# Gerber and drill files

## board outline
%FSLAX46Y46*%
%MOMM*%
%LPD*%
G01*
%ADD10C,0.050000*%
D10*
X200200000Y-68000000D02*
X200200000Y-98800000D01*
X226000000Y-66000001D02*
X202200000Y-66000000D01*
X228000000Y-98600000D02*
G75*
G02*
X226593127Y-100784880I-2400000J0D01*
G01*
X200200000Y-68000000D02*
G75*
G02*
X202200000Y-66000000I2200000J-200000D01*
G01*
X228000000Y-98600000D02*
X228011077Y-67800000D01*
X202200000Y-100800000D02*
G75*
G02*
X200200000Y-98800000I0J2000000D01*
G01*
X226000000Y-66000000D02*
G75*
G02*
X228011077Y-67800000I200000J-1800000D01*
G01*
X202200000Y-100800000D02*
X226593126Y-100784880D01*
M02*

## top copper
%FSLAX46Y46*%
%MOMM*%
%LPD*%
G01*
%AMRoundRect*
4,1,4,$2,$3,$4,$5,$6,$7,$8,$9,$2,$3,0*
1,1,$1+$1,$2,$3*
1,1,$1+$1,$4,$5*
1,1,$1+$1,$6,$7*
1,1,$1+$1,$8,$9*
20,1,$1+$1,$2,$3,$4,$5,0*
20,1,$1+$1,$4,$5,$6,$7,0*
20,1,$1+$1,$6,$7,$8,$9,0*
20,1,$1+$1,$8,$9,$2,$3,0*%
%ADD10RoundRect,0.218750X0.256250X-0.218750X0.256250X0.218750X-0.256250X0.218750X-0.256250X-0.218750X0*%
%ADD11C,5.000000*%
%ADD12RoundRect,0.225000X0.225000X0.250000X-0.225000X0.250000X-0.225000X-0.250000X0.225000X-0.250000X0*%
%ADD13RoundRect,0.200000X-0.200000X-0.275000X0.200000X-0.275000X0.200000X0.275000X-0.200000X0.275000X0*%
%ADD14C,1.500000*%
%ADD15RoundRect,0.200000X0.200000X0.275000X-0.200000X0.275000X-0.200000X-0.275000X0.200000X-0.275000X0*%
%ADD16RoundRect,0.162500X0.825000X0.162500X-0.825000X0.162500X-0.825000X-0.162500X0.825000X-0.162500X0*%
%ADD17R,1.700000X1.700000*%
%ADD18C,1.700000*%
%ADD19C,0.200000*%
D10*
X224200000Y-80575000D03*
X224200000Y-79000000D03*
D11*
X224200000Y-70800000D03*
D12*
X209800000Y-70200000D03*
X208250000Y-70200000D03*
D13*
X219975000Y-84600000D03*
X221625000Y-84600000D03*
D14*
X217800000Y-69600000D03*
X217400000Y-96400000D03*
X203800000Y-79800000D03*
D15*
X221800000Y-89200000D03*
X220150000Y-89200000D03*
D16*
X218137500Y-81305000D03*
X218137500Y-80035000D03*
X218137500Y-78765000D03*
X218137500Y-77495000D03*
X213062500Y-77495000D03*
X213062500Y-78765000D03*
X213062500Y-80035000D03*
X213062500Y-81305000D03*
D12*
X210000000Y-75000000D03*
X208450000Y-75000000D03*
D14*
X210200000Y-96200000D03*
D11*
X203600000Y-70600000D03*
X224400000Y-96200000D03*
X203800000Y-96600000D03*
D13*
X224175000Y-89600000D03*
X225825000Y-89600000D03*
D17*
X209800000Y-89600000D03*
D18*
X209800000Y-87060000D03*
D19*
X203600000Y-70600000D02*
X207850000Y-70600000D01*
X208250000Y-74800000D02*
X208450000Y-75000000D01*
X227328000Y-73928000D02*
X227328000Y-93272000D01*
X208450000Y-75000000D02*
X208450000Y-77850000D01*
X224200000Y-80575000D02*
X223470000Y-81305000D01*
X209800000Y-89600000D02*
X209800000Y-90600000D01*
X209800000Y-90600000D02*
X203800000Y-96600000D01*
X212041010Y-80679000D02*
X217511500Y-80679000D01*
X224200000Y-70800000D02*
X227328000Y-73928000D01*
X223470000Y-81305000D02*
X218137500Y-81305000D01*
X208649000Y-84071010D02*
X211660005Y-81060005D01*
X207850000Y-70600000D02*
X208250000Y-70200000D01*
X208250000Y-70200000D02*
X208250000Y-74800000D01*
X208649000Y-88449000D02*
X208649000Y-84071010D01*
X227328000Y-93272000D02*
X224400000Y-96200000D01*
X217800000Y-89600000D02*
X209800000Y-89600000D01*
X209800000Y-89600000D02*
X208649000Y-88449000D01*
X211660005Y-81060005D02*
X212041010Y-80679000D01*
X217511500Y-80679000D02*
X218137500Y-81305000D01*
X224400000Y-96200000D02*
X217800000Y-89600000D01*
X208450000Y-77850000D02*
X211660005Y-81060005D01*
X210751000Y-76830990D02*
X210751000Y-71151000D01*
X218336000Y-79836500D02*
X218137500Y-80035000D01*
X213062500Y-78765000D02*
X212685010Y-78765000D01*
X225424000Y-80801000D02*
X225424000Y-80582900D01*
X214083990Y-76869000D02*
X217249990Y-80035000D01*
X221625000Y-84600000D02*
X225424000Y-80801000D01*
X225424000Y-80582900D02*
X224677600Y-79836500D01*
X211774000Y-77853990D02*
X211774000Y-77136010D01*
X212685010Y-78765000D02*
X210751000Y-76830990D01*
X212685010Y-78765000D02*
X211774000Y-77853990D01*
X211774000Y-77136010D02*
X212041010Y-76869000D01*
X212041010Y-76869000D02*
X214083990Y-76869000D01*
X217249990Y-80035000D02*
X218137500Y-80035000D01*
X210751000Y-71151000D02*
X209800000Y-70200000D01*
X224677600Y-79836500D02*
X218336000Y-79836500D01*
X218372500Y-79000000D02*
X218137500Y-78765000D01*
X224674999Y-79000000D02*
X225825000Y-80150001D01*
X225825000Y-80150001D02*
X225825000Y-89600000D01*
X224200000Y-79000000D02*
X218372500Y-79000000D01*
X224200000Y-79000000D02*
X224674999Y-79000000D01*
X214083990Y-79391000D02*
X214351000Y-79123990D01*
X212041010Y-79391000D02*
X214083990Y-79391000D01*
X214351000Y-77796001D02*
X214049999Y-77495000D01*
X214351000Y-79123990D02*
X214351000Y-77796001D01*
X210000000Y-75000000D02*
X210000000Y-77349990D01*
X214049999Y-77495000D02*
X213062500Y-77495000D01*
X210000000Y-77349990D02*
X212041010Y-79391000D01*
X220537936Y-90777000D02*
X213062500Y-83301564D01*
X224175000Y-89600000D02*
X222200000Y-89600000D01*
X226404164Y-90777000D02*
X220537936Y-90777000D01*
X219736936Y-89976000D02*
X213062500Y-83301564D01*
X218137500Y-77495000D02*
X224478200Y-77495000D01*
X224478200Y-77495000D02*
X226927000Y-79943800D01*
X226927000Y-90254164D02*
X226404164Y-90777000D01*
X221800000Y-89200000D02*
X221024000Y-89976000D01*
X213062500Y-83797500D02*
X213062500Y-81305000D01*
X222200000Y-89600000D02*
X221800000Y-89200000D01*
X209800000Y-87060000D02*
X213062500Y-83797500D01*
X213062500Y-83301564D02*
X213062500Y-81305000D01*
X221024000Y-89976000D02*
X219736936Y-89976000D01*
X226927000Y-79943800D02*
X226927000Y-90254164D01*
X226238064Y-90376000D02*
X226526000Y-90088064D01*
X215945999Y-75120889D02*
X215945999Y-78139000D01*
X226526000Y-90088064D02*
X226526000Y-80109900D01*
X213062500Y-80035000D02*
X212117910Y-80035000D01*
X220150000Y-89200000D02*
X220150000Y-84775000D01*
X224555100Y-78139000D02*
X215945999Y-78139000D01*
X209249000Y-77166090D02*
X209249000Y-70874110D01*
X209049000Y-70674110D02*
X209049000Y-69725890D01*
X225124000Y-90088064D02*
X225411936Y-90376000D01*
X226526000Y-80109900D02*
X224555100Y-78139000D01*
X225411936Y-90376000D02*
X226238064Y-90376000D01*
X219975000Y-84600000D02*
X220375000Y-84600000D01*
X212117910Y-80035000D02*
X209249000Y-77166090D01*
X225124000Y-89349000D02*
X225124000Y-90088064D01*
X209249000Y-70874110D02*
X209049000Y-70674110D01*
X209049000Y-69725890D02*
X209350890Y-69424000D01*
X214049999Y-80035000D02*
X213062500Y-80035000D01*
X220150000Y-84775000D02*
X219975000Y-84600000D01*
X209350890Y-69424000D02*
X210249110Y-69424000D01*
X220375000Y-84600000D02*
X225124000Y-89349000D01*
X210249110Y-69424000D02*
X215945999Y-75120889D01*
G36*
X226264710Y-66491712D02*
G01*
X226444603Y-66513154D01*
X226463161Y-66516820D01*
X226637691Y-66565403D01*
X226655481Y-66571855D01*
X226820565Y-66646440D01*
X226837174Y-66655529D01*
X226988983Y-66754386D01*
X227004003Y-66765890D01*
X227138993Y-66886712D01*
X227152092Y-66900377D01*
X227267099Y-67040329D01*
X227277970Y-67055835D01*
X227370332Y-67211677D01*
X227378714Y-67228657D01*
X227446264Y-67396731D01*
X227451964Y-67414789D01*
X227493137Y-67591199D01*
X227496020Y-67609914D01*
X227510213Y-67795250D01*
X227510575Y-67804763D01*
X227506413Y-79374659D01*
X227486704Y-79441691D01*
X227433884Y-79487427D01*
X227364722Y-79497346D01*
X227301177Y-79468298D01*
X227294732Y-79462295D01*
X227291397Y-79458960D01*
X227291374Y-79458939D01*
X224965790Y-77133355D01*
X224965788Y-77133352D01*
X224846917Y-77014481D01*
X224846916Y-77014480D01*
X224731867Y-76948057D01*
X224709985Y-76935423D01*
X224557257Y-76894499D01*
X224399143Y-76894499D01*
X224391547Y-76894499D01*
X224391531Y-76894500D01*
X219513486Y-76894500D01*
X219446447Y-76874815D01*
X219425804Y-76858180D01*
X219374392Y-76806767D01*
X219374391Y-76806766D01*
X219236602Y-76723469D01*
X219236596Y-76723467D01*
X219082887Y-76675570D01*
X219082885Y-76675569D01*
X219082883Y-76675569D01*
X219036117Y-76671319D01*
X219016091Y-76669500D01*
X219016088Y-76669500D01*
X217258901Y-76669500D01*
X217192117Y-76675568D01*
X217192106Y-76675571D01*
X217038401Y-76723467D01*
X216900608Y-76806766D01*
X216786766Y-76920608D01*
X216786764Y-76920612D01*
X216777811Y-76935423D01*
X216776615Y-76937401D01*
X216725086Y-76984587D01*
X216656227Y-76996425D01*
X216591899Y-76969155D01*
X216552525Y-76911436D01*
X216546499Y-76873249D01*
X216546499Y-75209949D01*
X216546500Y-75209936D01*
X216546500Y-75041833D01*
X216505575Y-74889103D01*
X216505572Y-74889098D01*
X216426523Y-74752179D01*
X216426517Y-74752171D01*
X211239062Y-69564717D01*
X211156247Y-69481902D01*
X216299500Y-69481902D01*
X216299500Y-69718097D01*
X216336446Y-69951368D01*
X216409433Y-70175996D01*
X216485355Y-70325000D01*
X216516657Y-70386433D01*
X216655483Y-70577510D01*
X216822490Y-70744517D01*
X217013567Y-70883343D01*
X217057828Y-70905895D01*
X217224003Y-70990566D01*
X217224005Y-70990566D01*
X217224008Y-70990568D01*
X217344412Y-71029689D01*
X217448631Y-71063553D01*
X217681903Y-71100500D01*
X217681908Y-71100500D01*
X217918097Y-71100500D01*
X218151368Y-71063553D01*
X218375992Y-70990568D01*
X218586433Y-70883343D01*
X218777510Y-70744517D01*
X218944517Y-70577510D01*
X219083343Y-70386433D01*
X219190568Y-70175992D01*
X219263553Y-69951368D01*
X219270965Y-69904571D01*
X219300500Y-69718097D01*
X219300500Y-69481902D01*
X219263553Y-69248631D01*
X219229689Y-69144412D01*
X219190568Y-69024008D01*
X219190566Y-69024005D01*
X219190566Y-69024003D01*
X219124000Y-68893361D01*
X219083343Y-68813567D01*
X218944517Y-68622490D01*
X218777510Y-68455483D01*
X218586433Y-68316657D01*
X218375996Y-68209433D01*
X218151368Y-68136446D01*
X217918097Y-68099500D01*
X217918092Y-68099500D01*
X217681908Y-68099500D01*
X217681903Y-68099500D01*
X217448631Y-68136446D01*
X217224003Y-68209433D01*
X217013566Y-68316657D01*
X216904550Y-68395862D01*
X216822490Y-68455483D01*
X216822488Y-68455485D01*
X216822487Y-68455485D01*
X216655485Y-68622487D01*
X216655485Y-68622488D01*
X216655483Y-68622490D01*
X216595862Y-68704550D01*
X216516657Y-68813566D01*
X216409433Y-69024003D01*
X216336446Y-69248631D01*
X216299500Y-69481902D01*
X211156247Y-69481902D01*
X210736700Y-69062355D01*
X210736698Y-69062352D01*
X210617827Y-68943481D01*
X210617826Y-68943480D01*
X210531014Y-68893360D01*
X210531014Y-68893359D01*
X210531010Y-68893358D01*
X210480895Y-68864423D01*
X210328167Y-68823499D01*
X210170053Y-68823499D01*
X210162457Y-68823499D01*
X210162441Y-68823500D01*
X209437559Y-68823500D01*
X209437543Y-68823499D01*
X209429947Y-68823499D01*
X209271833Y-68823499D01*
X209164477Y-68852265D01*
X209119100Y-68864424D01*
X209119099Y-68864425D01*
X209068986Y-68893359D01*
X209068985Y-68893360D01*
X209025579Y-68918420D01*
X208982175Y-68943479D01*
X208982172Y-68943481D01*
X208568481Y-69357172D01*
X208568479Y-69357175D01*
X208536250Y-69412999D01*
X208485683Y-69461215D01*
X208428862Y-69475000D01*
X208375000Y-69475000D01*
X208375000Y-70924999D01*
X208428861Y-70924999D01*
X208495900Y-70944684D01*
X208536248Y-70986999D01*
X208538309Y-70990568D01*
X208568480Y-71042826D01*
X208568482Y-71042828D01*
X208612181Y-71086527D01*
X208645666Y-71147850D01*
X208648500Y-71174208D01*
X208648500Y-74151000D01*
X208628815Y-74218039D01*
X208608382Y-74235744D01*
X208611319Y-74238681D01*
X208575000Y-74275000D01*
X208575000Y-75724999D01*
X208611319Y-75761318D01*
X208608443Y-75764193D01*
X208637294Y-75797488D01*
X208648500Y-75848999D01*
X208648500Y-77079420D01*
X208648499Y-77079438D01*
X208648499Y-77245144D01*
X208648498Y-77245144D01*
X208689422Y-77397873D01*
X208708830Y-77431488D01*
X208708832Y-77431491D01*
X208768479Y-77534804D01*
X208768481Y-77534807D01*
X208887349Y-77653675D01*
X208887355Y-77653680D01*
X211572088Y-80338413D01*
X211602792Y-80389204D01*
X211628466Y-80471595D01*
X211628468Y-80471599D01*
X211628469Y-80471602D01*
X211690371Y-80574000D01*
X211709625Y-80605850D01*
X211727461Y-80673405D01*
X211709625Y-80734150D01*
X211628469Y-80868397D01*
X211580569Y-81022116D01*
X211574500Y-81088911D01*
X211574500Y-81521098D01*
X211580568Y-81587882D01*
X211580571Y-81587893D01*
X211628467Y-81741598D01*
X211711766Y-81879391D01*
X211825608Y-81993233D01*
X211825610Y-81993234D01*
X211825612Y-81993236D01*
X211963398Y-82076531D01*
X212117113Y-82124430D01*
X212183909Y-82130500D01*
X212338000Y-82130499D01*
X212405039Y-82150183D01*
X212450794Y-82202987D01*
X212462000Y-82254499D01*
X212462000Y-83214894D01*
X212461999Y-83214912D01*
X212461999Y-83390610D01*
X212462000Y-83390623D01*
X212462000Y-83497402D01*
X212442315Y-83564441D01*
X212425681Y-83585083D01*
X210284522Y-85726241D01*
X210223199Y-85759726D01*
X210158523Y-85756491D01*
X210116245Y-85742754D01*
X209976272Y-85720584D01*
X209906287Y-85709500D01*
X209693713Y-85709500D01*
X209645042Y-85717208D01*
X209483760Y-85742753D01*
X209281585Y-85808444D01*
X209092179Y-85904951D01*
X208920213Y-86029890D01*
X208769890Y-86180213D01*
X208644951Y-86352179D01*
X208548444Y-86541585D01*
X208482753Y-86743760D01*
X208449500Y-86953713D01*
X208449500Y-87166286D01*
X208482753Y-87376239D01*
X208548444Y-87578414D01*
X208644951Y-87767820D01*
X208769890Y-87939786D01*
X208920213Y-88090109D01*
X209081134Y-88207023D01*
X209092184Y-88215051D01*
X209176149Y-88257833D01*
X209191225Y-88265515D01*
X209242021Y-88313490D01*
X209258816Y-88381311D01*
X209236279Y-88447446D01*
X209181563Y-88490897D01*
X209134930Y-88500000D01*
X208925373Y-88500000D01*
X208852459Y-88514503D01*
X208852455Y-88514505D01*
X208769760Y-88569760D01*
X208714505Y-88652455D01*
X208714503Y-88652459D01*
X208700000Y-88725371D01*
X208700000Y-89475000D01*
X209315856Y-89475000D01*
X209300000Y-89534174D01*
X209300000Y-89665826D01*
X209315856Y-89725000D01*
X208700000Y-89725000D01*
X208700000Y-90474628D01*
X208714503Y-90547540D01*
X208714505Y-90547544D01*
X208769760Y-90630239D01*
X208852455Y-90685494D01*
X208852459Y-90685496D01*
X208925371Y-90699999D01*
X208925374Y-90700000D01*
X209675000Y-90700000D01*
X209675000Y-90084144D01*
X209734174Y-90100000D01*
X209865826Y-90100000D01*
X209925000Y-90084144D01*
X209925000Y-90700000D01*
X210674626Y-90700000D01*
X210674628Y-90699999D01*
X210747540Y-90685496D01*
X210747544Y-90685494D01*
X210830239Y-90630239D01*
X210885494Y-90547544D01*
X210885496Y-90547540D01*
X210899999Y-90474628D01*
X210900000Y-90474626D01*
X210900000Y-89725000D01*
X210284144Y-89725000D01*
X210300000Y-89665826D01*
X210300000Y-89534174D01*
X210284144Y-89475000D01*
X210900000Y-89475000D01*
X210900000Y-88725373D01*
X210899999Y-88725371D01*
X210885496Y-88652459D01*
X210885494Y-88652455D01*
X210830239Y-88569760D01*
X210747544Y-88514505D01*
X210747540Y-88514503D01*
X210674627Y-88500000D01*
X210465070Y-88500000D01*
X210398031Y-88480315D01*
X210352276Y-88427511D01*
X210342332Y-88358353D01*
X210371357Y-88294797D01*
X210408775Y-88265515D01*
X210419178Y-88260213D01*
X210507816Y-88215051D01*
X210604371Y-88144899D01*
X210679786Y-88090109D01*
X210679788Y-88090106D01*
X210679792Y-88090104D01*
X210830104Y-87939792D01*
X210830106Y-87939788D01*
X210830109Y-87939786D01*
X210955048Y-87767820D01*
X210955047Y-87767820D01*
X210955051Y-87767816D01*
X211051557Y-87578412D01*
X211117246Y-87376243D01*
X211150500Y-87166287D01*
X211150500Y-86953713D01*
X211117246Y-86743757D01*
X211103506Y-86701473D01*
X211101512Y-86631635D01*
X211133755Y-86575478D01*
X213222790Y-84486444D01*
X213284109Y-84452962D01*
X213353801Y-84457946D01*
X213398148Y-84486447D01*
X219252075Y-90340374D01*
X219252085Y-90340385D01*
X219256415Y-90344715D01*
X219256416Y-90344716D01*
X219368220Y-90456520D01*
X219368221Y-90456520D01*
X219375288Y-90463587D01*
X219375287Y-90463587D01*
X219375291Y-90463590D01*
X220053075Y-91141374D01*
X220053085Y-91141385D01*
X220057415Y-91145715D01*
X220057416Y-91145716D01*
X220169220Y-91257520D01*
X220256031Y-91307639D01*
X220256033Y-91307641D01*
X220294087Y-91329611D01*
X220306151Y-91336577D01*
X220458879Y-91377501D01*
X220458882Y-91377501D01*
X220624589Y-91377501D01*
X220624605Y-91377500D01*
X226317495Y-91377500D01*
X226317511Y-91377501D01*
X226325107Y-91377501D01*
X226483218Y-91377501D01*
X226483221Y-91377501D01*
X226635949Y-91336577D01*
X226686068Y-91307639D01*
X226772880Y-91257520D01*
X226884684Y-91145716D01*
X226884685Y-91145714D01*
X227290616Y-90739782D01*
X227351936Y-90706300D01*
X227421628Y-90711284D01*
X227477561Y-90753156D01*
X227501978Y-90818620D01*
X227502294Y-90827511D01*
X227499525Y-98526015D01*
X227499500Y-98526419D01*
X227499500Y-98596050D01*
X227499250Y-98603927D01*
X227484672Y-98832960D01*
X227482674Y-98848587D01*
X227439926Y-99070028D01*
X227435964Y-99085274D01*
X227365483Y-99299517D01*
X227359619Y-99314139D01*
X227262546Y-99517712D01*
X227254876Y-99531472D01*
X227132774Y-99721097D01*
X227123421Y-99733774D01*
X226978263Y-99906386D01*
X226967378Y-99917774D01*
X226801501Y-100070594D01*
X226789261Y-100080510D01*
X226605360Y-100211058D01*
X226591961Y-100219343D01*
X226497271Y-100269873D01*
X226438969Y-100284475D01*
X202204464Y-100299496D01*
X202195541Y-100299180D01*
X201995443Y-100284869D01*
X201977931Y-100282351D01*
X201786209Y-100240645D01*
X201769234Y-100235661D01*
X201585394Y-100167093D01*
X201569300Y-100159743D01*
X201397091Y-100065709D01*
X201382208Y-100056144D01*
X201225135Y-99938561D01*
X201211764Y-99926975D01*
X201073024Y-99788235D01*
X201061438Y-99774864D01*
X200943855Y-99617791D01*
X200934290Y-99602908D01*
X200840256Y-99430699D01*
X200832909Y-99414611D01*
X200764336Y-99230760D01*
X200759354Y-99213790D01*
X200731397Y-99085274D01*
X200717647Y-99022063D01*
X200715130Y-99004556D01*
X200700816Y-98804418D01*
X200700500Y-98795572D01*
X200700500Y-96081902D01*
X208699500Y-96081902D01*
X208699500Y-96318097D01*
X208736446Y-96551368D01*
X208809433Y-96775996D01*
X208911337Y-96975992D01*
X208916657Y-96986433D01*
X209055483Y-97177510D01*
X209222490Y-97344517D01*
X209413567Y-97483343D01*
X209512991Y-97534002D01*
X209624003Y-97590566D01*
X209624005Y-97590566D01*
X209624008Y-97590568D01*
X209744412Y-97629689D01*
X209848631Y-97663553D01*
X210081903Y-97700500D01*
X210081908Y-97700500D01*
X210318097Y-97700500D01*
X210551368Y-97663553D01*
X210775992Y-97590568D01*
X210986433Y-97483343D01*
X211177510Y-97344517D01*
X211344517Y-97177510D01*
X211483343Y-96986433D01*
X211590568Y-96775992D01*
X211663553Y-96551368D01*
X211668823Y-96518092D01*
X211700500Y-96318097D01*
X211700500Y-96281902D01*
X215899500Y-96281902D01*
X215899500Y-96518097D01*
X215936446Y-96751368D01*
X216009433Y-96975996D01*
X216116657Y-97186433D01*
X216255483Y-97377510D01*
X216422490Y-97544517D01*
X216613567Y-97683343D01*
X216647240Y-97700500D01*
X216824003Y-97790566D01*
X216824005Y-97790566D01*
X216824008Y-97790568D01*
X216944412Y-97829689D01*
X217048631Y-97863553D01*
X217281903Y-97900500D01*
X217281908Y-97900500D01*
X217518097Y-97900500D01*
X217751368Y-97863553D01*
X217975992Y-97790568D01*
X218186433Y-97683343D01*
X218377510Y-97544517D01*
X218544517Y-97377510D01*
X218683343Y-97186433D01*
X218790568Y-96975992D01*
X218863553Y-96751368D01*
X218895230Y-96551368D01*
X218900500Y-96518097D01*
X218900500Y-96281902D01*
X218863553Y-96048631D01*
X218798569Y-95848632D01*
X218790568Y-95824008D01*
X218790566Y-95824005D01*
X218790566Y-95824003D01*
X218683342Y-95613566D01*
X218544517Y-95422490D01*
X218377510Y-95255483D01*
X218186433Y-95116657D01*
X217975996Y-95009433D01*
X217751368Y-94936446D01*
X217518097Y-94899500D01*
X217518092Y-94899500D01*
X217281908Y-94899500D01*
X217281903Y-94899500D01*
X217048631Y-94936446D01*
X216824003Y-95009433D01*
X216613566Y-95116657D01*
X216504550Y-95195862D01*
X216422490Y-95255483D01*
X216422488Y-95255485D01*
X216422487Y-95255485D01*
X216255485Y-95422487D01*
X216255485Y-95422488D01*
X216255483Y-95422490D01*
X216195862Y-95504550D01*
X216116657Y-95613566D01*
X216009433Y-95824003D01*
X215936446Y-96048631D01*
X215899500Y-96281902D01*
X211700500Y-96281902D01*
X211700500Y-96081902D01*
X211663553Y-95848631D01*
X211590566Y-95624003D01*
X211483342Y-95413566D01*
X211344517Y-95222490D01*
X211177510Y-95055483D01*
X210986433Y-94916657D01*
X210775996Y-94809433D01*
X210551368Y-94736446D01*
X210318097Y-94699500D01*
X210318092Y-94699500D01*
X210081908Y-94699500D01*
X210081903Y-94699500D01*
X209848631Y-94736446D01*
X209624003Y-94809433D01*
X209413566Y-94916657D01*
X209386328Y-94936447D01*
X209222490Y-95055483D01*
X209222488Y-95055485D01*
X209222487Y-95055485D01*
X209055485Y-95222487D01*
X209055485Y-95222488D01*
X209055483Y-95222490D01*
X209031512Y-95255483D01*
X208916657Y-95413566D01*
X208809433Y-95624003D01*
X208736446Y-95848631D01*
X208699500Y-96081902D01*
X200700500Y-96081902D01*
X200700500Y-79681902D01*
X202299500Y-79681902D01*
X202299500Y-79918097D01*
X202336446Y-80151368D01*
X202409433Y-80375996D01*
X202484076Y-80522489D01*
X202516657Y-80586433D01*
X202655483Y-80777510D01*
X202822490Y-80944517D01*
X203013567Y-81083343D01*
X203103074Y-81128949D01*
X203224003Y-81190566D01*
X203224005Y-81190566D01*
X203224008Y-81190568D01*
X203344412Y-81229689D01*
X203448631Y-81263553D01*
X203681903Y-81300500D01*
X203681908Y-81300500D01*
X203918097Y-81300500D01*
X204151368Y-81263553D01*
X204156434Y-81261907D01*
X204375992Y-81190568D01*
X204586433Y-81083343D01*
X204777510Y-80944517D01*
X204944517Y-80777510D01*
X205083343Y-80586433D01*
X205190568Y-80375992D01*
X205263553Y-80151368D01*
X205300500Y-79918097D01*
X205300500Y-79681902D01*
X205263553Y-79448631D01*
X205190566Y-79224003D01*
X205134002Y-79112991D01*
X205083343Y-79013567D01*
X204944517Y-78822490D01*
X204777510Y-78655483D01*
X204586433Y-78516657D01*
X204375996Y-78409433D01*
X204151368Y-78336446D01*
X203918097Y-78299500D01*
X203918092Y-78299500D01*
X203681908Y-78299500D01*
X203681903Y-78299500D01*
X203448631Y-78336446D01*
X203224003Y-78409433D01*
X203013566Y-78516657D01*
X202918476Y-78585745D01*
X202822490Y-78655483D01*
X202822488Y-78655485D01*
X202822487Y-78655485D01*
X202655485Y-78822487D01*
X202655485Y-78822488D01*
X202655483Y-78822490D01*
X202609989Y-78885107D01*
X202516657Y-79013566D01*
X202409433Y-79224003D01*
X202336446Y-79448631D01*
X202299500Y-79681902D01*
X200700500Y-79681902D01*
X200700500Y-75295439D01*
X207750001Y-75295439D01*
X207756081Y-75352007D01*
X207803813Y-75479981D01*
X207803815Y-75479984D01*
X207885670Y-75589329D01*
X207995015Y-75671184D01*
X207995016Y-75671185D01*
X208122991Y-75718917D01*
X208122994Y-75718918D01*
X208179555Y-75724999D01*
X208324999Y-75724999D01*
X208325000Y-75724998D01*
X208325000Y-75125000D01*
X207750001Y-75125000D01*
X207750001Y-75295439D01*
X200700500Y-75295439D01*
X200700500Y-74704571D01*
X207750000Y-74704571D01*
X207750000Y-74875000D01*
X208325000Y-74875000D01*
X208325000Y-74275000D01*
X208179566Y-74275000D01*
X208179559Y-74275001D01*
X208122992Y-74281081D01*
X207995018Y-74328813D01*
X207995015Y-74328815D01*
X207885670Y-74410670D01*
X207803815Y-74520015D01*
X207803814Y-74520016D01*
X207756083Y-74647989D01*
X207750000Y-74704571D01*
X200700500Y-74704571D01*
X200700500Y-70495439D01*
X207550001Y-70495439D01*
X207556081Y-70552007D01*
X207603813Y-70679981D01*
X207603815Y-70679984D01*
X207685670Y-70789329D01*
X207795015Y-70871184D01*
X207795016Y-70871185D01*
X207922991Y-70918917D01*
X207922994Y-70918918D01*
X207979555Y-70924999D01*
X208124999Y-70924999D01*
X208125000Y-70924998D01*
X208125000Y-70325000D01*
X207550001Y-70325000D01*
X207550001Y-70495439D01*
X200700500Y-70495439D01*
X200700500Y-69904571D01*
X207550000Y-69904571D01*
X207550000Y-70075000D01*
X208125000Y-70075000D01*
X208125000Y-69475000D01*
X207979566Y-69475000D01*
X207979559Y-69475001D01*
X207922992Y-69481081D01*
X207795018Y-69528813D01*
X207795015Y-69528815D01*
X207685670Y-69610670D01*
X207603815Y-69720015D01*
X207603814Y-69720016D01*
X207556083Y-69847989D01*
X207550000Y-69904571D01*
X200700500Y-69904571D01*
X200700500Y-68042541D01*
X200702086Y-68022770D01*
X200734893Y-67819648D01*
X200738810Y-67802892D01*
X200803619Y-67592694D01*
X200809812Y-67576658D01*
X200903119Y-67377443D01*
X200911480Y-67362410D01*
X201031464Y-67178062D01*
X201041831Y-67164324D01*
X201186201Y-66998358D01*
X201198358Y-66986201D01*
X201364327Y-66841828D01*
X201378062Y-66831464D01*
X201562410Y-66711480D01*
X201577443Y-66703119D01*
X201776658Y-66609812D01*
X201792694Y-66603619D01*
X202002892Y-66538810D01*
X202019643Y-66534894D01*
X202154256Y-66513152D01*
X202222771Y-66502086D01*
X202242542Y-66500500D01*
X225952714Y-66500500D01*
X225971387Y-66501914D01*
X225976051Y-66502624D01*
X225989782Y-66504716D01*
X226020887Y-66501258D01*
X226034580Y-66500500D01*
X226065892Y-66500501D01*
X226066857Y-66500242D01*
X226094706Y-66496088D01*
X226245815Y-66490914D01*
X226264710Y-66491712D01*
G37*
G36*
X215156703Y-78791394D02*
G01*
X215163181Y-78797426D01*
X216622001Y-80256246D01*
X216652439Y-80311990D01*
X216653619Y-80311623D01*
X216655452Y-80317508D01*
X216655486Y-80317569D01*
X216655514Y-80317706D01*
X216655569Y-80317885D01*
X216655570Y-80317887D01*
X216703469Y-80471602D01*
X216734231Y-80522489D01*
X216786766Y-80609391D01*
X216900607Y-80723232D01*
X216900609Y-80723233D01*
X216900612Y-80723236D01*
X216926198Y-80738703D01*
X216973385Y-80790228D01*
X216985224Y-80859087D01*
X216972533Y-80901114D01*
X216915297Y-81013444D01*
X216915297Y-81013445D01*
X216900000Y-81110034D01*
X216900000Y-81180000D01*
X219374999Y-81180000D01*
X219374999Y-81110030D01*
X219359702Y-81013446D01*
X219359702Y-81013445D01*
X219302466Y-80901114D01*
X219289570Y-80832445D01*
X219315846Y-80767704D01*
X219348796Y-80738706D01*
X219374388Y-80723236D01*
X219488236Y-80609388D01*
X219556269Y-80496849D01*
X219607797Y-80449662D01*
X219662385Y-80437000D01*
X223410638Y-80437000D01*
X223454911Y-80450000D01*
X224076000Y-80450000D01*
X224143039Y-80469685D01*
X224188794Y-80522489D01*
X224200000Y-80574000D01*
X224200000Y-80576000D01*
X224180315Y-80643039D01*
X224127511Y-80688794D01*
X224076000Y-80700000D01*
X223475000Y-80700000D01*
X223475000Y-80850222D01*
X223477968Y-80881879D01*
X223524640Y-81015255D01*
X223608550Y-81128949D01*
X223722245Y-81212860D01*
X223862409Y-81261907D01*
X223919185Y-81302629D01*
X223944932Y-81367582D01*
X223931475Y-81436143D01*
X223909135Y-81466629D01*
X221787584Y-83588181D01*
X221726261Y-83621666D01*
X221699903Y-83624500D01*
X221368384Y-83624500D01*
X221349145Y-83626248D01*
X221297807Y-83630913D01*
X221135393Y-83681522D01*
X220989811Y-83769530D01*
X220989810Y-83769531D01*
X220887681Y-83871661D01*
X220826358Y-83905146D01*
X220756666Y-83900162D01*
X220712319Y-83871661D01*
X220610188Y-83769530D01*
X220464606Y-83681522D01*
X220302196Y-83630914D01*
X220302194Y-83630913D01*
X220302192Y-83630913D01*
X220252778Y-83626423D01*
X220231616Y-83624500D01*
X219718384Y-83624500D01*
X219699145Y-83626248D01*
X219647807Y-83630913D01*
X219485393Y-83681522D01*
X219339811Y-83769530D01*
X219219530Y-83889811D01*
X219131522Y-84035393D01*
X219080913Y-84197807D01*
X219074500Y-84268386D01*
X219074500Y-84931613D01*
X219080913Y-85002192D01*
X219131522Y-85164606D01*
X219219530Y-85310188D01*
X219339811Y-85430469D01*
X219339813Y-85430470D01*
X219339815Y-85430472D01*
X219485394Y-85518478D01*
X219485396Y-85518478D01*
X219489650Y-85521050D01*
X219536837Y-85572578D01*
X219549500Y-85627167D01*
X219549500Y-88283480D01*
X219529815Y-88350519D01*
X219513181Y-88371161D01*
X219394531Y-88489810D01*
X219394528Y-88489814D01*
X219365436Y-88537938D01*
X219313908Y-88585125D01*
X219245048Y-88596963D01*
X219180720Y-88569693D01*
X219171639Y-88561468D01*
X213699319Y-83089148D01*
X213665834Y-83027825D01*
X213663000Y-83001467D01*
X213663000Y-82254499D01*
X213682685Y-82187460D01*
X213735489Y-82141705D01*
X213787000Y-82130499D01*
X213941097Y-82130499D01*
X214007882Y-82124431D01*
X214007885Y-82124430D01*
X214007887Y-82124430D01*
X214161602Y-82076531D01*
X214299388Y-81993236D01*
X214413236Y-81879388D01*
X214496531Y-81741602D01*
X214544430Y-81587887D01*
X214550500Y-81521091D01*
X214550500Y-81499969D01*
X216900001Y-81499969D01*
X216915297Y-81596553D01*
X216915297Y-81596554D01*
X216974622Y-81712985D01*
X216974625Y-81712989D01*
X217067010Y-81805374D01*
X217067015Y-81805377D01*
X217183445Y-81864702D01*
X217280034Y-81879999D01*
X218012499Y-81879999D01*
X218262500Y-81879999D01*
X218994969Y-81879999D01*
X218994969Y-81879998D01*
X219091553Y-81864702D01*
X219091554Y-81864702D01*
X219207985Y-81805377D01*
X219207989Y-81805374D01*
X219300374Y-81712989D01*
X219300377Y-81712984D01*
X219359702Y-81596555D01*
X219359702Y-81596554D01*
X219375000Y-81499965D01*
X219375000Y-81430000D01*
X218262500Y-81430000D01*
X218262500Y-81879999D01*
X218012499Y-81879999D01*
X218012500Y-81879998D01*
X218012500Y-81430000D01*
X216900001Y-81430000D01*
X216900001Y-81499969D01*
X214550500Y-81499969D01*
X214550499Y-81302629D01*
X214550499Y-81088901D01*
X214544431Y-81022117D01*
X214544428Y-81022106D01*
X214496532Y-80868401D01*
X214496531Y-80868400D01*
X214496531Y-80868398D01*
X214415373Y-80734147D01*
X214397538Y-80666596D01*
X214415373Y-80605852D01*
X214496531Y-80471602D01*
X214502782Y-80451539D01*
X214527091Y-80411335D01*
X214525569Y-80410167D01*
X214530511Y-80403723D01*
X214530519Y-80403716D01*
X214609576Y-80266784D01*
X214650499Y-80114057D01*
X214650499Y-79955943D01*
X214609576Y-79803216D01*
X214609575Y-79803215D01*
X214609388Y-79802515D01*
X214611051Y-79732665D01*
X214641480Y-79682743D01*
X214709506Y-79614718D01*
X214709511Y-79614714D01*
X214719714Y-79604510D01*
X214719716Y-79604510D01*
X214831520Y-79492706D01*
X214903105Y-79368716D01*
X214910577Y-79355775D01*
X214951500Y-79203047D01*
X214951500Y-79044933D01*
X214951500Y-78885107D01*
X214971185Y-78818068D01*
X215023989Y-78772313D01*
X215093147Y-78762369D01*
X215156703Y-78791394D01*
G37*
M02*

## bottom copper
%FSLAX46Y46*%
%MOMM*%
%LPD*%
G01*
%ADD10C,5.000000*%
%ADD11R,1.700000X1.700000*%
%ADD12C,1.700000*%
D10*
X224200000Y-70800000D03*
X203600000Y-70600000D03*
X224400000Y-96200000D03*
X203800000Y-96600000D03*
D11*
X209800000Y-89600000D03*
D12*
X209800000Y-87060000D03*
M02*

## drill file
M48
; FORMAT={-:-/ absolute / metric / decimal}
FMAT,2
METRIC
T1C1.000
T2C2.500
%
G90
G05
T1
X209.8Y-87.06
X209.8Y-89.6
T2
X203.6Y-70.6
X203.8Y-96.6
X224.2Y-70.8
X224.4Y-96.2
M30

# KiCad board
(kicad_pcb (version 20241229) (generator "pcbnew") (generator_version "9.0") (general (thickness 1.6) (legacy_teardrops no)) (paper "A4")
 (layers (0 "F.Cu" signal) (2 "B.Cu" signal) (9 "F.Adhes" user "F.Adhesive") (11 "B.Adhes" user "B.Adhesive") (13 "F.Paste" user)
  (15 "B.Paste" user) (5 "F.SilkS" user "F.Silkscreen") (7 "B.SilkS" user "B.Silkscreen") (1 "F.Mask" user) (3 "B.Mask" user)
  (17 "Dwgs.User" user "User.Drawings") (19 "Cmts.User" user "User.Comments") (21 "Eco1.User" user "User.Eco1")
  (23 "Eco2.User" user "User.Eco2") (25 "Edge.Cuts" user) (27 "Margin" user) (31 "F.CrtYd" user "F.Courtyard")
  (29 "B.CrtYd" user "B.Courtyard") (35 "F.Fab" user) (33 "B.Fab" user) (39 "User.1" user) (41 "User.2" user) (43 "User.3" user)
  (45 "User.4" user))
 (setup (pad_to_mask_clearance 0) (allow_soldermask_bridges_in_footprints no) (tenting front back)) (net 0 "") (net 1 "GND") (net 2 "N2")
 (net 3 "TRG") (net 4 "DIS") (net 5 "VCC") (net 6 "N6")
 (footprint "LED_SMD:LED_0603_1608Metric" (layer "F.Cu") (at 224.2 79.7875 90)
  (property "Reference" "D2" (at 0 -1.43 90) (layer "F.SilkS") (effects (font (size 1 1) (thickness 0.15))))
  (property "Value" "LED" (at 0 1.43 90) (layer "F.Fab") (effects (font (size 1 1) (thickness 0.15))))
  (pad "1" smd roundrect (at -0.7875 0 90) (size 0.875 0.95) (layers "F.Cu" "F.Mask" "F.Paste") (roundrect_rratio 0.25) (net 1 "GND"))
  (pad "2" smd roundrect (at 0.7875 0 90) (size 0.875 0.95) (layers "F.Cu" "F.Mask" "F.Paste") (roundrect_rratio 0.25) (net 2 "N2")))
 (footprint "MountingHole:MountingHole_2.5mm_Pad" (layer "F.Cu") (at 224.2 70.8)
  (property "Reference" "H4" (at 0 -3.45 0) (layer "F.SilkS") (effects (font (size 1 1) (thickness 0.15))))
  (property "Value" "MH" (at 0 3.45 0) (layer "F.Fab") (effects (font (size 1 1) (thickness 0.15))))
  (pad "1" thru_hole circle (at 0 0) (size 5 5) (drill 2.5) (layers "*.Cu" "*.Mask") (remove_unused_layers no) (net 1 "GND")
   (zone_connect 2)))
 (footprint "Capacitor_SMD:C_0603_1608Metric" (layer "F.Cu") (at 209.025 70.2 180)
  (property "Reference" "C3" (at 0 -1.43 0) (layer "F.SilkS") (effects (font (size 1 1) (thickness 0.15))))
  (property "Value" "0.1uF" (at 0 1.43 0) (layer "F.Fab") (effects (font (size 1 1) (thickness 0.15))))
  (pad "1" smd roundrect (at -0.775 0 180) (size 0.9 0.95) (layers "F.Cu" "F.Mask" "F.Paste") (roundrect_rratio 0.25) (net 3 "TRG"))
  (pad "2" smd roundrect (at 0.775 0 180) (size 0.9 0.95) (layers "F.Cu" "F.Mask" "F.Paste") (roundrect_rratio 0.25) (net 1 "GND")))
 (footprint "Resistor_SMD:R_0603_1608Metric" (layer "F.Cu") (at 220.8 84.6)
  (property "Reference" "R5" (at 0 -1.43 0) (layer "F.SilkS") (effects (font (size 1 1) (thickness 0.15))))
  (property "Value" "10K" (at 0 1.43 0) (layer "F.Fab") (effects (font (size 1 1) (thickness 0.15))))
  (pad "1" smd roundrect (at -0.825 0) (size 0.8 0.95) (layers "F.Cu" "F.Mask" "F.Paste") (roundrect_rratio 0.25) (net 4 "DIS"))
  (pad "2" smd roundrect (at 0.825 0) (size 0.8 0.95) (layers "F.Cu" "F.Mask" "F.Paste") (roundrect_rratio 0.25) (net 3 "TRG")))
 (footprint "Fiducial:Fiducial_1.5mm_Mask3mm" (layer "F.Cu") (at 217.8 69.6)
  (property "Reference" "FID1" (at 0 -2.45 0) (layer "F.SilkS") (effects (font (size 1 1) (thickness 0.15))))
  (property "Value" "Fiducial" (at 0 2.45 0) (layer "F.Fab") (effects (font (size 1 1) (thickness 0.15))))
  (pad "" smd circle (at 0 0) (size 1.5 1.5) (layers "F.Cu" "F.Mask") (solder_mask_margin 0.75) (clearance 0.75)))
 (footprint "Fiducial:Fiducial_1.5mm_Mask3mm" (layer "F.Cu") (at 217.4 96.4)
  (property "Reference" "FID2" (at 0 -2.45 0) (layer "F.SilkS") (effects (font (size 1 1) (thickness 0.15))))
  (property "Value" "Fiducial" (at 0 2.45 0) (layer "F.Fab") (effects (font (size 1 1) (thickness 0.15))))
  (pad "" smd circle (at 0 0) (size 1.5 1.5) (layers "F.Cu" "F.Mask") (solder_mask_margin 0.75) (clearance 0.75)))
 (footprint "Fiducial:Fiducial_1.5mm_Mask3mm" (layer "F.Cu") (at 203.8 79.8)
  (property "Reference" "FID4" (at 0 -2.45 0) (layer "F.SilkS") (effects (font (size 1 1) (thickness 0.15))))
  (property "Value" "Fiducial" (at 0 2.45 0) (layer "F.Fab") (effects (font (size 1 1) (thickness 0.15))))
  (pad "" smd circle (at 0 0) (size 1.5 1.5) (layers "F.Cu" "F.Mask") (solder_mask_margin 0.75) (clearance 0.75)))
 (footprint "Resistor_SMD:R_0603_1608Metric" (layer "F.Cu") (at 220.975 89.2 180)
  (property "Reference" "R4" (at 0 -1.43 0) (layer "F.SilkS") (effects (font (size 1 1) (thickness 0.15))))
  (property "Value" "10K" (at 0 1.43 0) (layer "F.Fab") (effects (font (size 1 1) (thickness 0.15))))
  (pad "1" smd roundrect (at -0.825 0 180) (size 0.8 0.95) (layers "F.Cu" "F.Mask" "F.Paste") (roundrect_rratio 0.25) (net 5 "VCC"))
  (pad "2" smd roundrect (at 0.825 0 180) (size 0.8 0.95) (layers "F.Cu" "F.Mask" "F.Paste") (roundrect_rratio 0.25) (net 4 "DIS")))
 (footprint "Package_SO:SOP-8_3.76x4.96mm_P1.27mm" (layer "F.Cu") (at 215.6 79.4 180)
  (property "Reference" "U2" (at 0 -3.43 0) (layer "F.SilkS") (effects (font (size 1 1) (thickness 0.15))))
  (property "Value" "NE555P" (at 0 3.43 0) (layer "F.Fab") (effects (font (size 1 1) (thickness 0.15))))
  (pad "1" smd roundrect (at -2.5375 -1.905 180) (size 1.975 0.65) (layers "F.Cu" "F.Mask" "F.Paste") (roundrect_rratio 0.25) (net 1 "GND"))
  (pad "2" smd roundrect (at -2.5375 -0.635 180) (size 1.975 0.65) (layers "F.Cu" "F.Mask" "F.Paste") (roundrect_rratio 0.25) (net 3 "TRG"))
  (pad "3" smd roundrect (at -2.5375 0.635 180) (size 1.975 0.65) (layers "F.Cu" "F.Mask" "F.Paste") (roundrect_rratio 0.25) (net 2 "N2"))
  (pad "4" smd roundrect (at -2.5375 1.905 180) (size 1.975 0.65) (layers "F.Cu" "F.Mask" "F.Paste") (roundrect_rratio 0.25) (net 5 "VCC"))
  (pad "5" smd roundrect (at 2.5375 1.905 180) (size 1.975 0.65) (layers "F.Cu" "F.Mask" "F.Paste") (roundrect_rratio 0.25) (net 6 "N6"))
  (pad "6" smd roundrect (at 2.5375 0.635 180) (size 1.975 0.65) (layers "F.Cu" "F.Mask" "F.Paste") (roundrect_rratio 0.25) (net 3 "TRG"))
  (pad "7" smd roundrect (at 2.5375 -0.635 180) (size 1.975 0.65) (layers "F.Cu" "F.Mask" "F.Paste") (roundrect_rratio 0.25) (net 4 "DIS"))
  (pad "8" smd roundrect (at 2.5375 -1.905 180) (size 1.975 0.65) (layers "F.Cu" "F.Mask" "F.Paste") (roundrect_rratio 0.25) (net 5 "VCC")))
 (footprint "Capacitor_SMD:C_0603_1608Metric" (layer "F.Cu") (at 209.225 75 180)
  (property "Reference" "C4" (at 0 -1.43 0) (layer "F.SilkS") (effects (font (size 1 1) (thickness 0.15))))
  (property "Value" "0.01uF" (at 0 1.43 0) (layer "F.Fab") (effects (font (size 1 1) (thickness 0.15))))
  (pad "1" smd roundrect (at -0.775 0 180) (size 0.9 0.95) (layers "F.Cu" "F.Mask" "F.Paste") (roundrect_rratio 0.25) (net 6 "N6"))
  (pad "2" smd roundrect (at 0.775 0 180) (size 0.9 0.95) (layers "F.Cu" "F.Mask" "F.Paste") (roundrect_rratio 0.25) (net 1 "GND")))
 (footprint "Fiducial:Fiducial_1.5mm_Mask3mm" (layer "F.Cu") (at 210.2 96.2)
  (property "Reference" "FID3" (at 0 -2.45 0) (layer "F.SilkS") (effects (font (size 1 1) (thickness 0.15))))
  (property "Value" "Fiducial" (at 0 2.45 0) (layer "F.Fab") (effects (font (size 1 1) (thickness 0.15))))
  (pad "" smd circle (at 0 0) (size 1.5 1.5) (layers "F.Cu" "F.Mask") (solder_mask_margin 0.75) (clearance 0.75)))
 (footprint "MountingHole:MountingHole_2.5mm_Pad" (layer "F.Cu") (at 203.6 70.6)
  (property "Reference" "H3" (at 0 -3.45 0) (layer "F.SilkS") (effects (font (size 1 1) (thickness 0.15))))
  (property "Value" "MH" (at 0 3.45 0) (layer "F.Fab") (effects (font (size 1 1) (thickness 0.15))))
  (pad "1" thru_hole circle (at 0 0) (size 5 5) (drill 2.5) (layers "*.Cu" "*.Mask") (remove_unused_layers no) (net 1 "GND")
   (zone_connect 2)))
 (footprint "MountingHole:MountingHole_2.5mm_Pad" (layer "F.Cu") (at 224.4 96.2)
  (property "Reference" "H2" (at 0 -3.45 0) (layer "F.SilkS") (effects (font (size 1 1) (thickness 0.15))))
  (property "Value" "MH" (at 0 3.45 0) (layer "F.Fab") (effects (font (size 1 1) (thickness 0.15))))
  (pad "1" thru_hole circle (at 0 0) (size 5 5) (drill 2.5) (layers "*.Cu" "*.Mask") (remove_unused_layers no) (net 1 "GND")
   (zone_connect 2)))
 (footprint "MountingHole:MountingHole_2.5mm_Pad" (layer "F.Cu") (at 203.8 96.6)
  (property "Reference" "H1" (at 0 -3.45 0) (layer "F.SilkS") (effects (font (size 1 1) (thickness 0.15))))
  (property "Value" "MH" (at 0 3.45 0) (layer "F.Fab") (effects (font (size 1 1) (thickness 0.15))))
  (pad "1" thru_hole circle (at 0 0) (size 5 5) (drill 2.5) (layers "*.Cu" "*.Mask") (remove_unused_layers no) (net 1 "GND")
   (zone_connect 2)))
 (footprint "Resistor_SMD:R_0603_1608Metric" (layer "F.Cu") (at 225 89.6)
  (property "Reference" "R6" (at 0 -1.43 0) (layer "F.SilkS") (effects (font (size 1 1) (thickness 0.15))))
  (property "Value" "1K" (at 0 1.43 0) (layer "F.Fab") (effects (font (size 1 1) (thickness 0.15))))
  (pad "1" smd roundrect (at -0.825 0) (size 0.8 0.95) (layers "F.Cu" "F.Mask" "F.Paste") (roundrect_rratio 0.25) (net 5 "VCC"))
  (pad "2" smd roundrect (at 0.825 0) (size 0.8 0.95) (layers "F.Cu" "F.Mask" "F.Paste") (roundrect_rratio 0.25) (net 2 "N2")))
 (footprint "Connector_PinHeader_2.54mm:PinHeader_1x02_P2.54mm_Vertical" (layer "F.Cu") (at 209.8 89.6 180)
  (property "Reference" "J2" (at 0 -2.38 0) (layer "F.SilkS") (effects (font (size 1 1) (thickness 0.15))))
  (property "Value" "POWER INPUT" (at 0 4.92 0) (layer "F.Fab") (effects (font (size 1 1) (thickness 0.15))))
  (pad "1" thru_hole rect (at 0 0 180) (size 1.7 1.7) (drill 1) (layers "*.Cu" "*.Mask") (remove_unused_layers no) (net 1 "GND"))
  (pad "2" thru_hole circle (at 0 2.54 180) (size 1.7 1.7) (drill 1) (layers "*.Cu" "*.Mask") (remove_unused_layers no) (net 5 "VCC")))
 (gr_line (start 200.2 68) (end 200.2 98.8) (stroke (width 0.05) (type default)) (layer "Edge.Cuts"))
 (gr_line (start 226 66.000001) (end 202.2 66) (stroke (width 0.05) (type default)) (layer "Edge.Cuts"))
 (gr_arc (start 228 98.6) (mid 227.617858 99.899326) (end 226.593127 100.78488) (stroke (width 0.05) (type default)) (layer "Edge.Cuts"))
 (gr_arc (start 200.2 68) (mid 200.83795 66.63795) (end 202.2 66) (stroke (width 0.05) (type default)) (layer "Edge.Cuts"))
 (gr_line (start 228 98.6) (end 228.011077 67.8) (stroke (width 0.05) (type default)) (layer "Edge.Cuts"))
 (gr_arc (start 202.2 100.8) (mid 200.785786 100.214214) (end 200.2 98.8) (stroke (width 0.05) (type default)) (layer "Edge.Cuts"))
 (gr_arc (start 226 66) (mid 227.407846 66.450516) (end 228.011077 67.8) (stroke (width 0.05) (type default)) (layer "Edge.Cuts"))
 (gr_line (start 202.2 100.8) (end 226.593126 100.78488) (stroke (width 0.05) (type default)) (layer "Edge.Cuts"))
 (segment (start 203.6 70.6) (end 207.85 70.6) (width 0.2) (layer "F.Cu") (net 1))
 (segment (start 208.25 74.8) (end 208.45 75) (width 0.2) (layer "F.Cu") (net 1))
 (segment (start 227.328 73.928) (end 227.328 93.272) (width 0.2) (layer "F.Cu") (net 1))
 (segment (start 208.45 75) (end 208.45 77.85) (width 0.2) (layer "F.Cu") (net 1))
 (segment (start 224.2 80.575) (end 223.47 81.305) (width 0.2) (layer "F.Cu") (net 1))
 (segment (start 209.8 89.6) (end 209.8 90.6) (width 0.2) (layer "F.Cu") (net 1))
 (segment (start 209.8 90.6) (end 203.8 96.6) (width 0.2) (layer "F.Cu") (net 1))
 (segment (start 212.04101 80.679) (end 217.5115 80.679) (width 0.2) (layer "F.Cu") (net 1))
 (segment (start 224.2 70.8) (end 227.328 73.928) (width 0.2) (layer "F.Cu") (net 1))
 (segment (start 223.47 81.305) (end 218.1375 81.305) (width 0.2) (layer "F.Cu") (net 1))
 (segment (start 208.649 84.07101) (end 211.660005 81.060005) (width 0.2) (layer "F.Cu") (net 1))
 (segment (start 207.85 70.6) (end 208.25 70.2) (width 0.2) (layer "F.Cu") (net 1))
 (segment (start 208.25 70.2) (end 208.25 74.8) (width 0.2) (layer "F.Cu") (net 1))
 (segment (start 208.649 88.449) (end 208.649 84.07101) (width 0.2) (layer "F.Cu") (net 1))
 (segment (start 227.328 93.272) (end 224.4 96.2) (width 0.2) (layer "F.Cu") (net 1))
 (segment (start 217.8 89.6) (end 209.8 89.6) (width 0.2) (layer "F.Cu") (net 1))
 (segment (start 209.8 89.6) (end 208.649 88.449) (width 0.2) (layer "F.Cu") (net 1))
 (segment (start 211.660005 81.060005) (end 212.04101 80.679) (width 0.2) (layer "F.Cu") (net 1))
 (segment (start 217.5115 80.679) (end 218.1375 81.305) (width 0.2) (layer "F.Cu") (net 1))
 (segment (start 224.4 96.2) (end 217.8 89.6) (width 0.2) (layer "F.Cu") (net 1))
 (segment (start 208.45 77.85) (end 211.660005 81.060005) (width 0.2) (layer "F.Cu") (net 1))
 (segment (start 210.751 76.83099) (end 210.751 71.151) (width 0.2) (layer "F.Cu") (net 3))
 (segment (start 218.336 79.8365) (end 218.1375 80.035) (width 0.2) (layer "F.Cu") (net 3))
 (segment (start 213.0625 78.765) (end 212.68501 78.765) (width 0.2) (layer "F.Cu") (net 3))
 (segment (start 225.424 80.801) (end 225.424 80.5829) (width 0.2) (layer "F.Cu") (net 3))
 (segment (start 214.08399 76.869) (end 217.24999 80.035) (width 0.2) (layer "F.Cu") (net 3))
 (segment (start 221.625 84.6) (end 225.424 80.801) (width 0.2) (layer "F.Cu") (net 3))
 (segment (start 225.424 80.5829) (end 224.6776 79.8365) (width 0.2) (layer "F.Cu") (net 3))
 (segment (start 211.774 77.85399) (end 211.774 77.13601) (width 0.2) (layer "F.Cu") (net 3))
 (segment (start 212.68501 78.765) (end 210.751 76.83099) (width 0.2) (layer "F.Cu") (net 3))
 (segment (start 212.68501 78.765) (end 211.774 77.85399) (width 0.2) (layer "F.Cu") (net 3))
 (segment (start 211.774 77.13601) (end 212.04101 76.869) (width 0.2) (layer "F.Cu") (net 3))
 (segment (start 212.04101 76.869) (end 214.08399 76.869) (width 0.2) (layer "F.Cu") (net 3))
 (segment (start 217.24999 80.035) (end 218.1375 80.035) (width 0.2) (layer "F.Cu") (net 3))
 (segment (start 210.751 71.151) (end 209.8 70.2) (width 0.2) (layer "F.Cu") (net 3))
 (segment (start 224.6776 79.8365) (end 218.336 79.8365) (width 0.2) (layer "F.Cu") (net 3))
 (segment (start 218.3725 79) (end 218.1375 78.765) (width 0.2) (layer "F.Cu") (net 2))
 (segment (start 224.674999 79) (end 225.825 80.150001) (width 0.2) (layer "F.Cu") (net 2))
 (segment (start 225.825 80.150001) (end 225.825 89.6) (width 0.2) (layer "F.Cu") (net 2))
 (segment (start 224.2 79) (end 218.3725 79) (width 0.2) (layer "F.Cu") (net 2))
 (segment (start 224.2 79) (end 224.674999 79) (width 0.2) (layer "F.Cu") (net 2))
 (segment (start 214.08399 79.391) (end 214.351 79.12399) (width 0.2) (layer "F.Cu") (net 6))
 (segment (start 212.04101 79.391) (end 214.08399 79.391) (width 0.2) (layer "F.Cu") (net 6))
 (segment (start 214.351 77.796001) (end 214.049999 77.495) (width 0.2) (layer "F.Cu") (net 6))
 (segment (start 214.351 79.12399) (end 214.351 77.796001) (width 0.2) (layer "F.Cu") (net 6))
 (segment (start 210 75) (end 210 77.34999) (width 0.2) (layer "F.Cu") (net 6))
 (segment (start 214.049999 77.495) (end 213.0625 77.495) (width 0.2) (layer "F.Cu") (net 6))
 (segment (start 210 77.34999) (end 212.04101 79.391) (width 0.2) (layer "F.Cu") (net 6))
 (segment (start 220.537936 90.777) (end 213.0625 83.301564) (width 0.2) (layer "F.Cu") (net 5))
 (segment (start 224.175 89.6) (end 222.2 89.6) (width 0.2) (layer "F.Cu") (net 5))
 (segment (start 226.404164 90.777) (end 220.537936 90.777) (width 0.2) (layer "F.Cu") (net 5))
 (segment (start 219.736936 89.976) (end 213.0625 83.301564) (width 0.2) (layer "F.Cu") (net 5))
 (segment (start 218.1375 77.495) (end 224.4782 77.495) (width 0.2) (layer "F.Cu") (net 5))
 (segment (start 224.4782 77.495) (end 226.927 79.9438) (width 0.2) (layer "F.Cu") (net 5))
 (segment (start 226.927 90.254164) (end 226.404164 90.777) (width 0.2) (layer "F.Cu") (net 5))
 (segment (start 221.8 89.2) (end 221.024 89.976) (width 0.2) (layer "F.Cu") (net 5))
 (segment (start 213.0625 83.7975) (end 213.0625 81.305) (width 0.2) (layer "F.Cu") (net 5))
 (segment (start 222.2 89.6) (end 221.8 89.2) (width 0.2) (layer "F.Cu") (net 5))
 (segment (start 209.8 87.06) (end 213.0625 83.7975) (width 0.2) (layer "F.Cu") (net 5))
 (segment (start 213.0625 83.301564) (end 213.0625 81.305) (width 0.2) (layer "F.Cu") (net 5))
 (segment (start 221.024 89.976) (end 219.736936 89.976) (width 0.2) (layer "F.Cu") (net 5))
 (segment (start 226.927 79.9438) (end 226.927 90.254164) (width 0.2) (layer "F.Cu") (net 5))
 (segment (start 226.238064 90.376) (end 226.526 90.088064) (width 0.2) (layer "F.Cu") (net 4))
 (segment (start 215.945999 75.120889) (end 215.945999 78.139) (width 0.2) (layer "F.Cu") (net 4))
 (segment (start 226.526 90.088064) (end 226.526 80.1099) (width 0.2) (layer "F.Cu") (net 4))
 (segment (start 213.0625 80.035) (end 212.11791 80.035) (width 0.2) (layer "F.Cu") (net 4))
 (segment (start 220.15 89.2) (end 220.15 84.775) (width 0.2) (layer "F.Cu") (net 4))
 (segment (start 224.5551 78.139) (end 215.945999 78.139) (width 0.2) (layer "F.Cu") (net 4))
 (segment (start 209.249 77.16609) (end 209.249 70.87411) (width 0.2) (layer "F.Cu") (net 4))
 (segment (start 209.049 70.67411) (end 209.049 69.72589) (width 0.2) (layer "F.Cu") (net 4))
 (segment (start 225.124 90.088064) (end 225.411936 90.376) (width 0.2) (layer "F.Cu") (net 4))
 (segment (start 226.526 80.1099) (end 224.5551 78.139) (width 0.2) (layer "F.Cu") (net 4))
 (segment (start 225.411936 90.376) (end 226.238064 90.376) (width 0.2) (layer "F.Cu") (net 4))
 (segment (start 219.975 84.6) (end 220.375 84.6) (width 0.2) (layer "F.Cu") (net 4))
 (segment (start 212.11791 80.035) (end 209.249 77.16609) (width 0.2) (layer "F.Cu") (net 4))
 (segment (start 225.124 89.349) (end 225.124 90.088064) (width 0.2) (layer "F.Cu") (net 4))
 (segment (start 209.249 70.87411) (end 209.049 70.67411) (width 0.2) (layer "F.Cu") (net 4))
 (segment (start 209.049 69.72589) (end 209.35089 69.424) (width 0.2) (layer "F.Cu") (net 4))
 (segment (start 214.049999 80.035) (end 213.0625 80.035) (width 0.2) (layer "F.Cu") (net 4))
 (segment (start 220.15 84.775) (end 219.975 84.6) (width 0.2) (layer "F.Cu") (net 4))
 (segment (start 209.35089 69.424) (end 210.24911 69.424) (width 0.2) (layer "F.Cu") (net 4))
 (segment (start 220.375 84.6) (end 225.124 89.349) (width 0.2) (layer "F.Cu") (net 4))
 (segment (start 210.24911 69.424) (end 215.945999 75.120889) (width 0.2) (layer "F.Cu") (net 4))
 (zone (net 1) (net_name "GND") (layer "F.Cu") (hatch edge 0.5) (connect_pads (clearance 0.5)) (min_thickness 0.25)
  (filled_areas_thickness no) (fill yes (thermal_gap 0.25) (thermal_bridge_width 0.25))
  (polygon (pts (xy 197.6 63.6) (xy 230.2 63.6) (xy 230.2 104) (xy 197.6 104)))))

